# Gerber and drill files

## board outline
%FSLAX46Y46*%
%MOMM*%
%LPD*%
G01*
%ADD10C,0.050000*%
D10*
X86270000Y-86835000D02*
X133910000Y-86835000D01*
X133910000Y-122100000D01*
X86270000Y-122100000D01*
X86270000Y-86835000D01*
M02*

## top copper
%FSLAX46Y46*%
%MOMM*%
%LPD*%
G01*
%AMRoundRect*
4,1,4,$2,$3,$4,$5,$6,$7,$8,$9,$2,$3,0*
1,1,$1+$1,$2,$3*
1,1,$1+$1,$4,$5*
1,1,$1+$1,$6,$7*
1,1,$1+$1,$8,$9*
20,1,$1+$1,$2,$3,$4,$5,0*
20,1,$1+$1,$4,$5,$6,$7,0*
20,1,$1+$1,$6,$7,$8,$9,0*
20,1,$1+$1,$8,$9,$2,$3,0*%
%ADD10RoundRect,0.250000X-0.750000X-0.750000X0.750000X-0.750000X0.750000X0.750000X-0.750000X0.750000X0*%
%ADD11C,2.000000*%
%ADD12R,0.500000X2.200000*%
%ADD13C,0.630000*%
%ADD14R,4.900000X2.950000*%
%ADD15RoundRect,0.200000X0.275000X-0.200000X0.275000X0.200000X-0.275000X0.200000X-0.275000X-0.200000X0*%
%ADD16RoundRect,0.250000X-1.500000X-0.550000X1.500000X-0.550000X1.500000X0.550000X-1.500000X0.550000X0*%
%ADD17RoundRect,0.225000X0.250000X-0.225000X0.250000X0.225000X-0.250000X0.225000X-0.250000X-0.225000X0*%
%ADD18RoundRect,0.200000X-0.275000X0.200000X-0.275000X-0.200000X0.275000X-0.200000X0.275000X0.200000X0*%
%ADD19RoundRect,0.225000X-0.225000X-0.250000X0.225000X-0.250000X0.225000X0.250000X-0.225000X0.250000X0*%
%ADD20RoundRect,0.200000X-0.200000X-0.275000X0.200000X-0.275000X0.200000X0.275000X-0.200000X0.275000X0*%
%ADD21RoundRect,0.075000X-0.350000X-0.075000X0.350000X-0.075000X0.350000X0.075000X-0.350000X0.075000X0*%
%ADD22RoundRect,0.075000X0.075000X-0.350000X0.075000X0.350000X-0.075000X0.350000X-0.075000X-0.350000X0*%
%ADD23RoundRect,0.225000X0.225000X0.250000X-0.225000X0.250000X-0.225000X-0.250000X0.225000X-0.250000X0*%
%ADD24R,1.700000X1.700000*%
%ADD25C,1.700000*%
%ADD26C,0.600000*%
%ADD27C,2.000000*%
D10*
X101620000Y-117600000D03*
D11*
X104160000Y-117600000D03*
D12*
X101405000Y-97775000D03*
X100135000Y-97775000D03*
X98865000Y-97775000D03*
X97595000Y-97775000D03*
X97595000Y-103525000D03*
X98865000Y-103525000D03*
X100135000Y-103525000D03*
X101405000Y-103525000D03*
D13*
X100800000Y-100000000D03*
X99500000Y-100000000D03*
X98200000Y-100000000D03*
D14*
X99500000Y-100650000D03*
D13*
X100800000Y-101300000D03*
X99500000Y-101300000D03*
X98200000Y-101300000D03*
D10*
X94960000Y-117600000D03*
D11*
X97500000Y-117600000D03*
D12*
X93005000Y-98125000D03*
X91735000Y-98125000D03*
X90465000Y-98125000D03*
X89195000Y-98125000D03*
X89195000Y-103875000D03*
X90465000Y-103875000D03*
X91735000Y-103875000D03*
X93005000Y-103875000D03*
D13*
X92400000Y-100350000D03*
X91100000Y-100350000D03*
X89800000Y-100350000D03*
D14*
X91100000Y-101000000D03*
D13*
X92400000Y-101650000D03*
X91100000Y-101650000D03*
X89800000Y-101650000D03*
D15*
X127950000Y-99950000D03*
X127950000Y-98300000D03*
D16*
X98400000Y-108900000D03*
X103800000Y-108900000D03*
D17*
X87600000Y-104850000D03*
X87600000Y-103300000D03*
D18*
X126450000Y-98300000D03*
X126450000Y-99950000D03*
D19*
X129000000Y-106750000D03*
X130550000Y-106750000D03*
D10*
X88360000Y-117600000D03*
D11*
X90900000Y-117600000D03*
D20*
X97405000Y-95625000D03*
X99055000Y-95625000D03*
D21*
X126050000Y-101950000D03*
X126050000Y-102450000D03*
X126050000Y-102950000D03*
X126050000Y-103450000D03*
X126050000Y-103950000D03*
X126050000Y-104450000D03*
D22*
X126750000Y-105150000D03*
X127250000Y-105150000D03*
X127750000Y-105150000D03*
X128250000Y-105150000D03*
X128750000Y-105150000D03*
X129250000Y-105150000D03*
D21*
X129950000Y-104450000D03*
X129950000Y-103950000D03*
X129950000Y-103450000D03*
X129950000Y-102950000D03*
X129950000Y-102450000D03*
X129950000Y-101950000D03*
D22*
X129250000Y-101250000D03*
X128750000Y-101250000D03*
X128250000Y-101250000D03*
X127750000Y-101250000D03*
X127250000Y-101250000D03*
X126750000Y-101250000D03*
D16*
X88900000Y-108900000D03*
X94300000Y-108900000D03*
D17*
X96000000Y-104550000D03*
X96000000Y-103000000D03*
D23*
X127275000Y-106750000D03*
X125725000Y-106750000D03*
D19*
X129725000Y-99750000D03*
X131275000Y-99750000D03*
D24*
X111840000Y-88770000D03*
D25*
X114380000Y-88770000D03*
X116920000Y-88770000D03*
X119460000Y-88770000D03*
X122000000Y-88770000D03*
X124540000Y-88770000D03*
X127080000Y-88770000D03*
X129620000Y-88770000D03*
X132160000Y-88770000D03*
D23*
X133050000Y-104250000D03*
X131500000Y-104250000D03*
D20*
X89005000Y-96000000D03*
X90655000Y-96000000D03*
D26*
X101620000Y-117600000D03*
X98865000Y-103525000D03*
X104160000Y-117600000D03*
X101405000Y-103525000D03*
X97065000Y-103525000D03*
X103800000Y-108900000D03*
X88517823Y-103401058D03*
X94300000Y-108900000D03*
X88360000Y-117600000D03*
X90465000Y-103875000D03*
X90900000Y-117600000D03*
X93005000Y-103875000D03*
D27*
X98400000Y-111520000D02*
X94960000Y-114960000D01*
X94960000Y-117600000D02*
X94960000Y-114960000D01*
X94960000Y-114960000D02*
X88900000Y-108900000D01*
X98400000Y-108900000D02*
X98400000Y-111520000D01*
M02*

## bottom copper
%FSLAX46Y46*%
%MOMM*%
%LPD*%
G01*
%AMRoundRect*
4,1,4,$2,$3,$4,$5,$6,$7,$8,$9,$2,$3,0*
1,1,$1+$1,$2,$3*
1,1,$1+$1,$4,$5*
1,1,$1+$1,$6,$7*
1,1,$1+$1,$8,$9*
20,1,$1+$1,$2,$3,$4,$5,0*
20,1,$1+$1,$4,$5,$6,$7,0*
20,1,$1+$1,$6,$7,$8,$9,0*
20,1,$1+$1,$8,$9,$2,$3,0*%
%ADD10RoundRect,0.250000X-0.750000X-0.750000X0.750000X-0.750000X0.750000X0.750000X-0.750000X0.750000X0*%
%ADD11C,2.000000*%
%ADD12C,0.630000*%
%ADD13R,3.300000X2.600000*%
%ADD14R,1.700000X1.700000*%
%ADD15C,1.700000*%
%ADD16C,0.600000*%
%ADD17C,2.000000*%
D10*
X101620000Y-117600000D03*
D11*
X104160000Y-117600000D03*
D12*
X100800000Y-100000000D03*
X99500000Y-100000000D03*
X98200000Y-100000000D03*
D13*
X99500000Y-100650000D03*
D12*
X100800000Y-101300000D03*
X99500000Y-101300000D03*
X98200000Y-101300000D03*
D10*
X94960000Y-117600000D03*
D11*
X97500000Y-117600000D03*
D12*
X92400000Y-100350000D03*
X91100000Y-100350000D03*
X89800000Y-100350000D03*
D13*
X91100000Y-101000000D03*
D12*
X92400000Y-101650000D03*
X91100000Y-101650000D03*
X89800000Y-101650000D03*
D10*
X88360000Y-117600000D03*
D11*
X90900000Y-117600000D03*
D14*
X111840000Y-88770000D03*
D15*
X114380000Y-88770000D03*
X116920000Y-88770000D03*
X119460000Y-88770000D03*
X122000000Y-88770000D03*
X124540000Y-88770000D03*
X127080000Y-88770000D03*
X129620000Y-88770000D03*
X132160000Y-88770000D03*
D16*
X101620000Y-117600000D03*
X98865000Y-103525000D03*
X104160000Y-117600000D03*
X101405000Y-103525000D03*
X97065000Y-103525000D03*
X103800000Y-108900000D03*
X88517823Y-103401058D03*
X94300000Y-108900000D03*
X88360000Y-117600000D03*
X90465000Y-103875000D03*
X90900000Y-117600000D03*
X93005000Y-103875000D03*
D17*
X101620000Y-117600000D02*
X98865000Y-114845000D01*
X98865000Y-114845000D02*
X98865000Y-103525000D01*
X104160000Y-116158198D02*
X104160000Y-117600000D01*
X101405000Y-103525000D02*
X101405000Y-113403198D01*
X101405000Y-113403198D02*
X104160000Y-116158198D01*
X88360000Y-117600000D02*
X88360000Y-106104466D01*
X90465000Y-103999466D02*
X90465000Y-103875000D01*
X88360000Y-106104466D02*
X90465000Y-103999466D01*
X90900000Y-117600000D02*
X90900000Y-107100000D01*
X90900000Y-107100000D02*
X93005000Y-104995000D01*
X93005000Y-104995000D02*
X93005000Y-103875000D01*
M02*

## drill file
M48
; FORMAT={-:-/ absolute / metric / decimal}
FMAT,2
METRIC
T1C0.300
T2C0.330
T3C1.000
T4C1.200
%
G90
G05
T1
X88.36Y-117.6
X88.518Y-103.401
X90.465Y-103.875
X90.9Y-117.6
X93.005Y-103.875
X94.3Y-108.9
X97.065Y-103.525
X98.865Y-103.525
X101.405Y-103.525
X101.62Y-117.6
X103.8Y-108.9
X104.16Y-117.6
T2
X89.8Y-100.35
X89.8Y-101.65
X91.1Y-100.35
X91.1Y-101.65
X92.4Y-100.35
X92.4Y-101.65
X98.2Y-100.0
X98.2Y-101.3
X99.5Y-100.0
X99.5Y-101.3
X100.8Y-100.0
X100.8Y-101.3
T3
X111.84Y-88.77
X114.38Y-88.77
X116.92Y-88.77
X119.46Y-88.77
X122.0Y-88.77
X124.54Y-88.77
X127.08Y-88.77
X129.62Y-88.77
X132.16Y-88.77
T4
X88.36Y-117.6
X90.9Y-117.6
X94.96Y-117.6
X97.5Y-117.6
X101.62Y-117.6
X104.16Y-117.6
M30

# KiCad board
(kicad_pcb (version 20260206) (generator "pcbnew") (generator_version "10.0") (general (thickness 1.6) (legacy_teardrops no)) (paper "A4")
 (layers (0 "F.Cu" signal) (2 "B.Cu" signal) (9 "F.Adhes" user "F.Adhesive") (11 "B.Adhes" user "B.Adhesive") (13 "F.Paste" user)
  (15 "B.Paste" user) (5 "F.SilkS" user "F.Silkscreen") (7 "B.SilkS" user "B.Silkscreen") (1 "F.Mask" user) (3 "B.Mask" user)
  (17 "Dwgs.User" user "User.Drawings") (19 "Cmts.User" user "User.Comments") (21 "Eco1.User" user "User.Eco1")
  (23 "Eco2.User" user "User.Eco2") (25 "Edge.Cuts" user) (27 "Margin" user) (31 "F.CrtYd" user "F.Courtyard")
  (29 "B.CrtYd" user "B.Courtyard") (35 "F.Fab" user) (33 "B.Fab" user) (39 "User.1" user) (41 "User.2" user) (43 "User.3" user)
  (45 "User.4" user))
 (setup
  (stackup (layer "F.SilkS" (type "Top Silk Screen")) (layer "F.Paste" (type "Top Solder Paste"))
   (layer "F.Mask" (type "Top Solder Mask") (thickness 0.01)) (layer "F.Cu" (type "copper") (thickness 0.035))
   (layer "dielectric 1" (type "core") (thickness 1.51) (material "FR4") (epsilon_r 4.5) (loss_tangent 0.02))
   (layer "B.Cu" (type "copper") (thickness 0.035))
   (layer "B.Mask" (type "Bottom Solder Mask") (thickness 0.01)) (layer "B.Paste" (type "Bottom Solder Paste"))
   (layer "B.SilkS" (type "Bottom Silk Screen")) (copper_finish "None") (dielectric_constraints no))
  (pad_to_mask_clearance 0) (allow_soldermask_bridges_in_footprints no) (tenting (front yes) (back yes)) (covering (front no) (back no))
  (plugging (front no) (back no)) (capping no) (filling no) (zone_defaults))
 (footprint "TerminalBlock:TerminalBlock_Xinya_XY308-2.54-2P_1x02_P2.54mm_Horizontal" (layer "F.Cu") (at 101.62 117.6)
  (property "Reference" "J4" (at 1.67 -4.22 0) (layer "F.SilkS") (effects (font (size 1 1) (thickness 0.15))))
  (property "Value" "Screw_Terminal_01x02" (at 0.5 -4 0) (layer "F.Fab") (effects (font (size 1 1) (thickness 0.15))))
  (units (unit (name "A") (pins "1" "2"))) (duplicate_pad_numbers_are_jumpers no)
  (pad "1" thru_hole roundrect (at 0 0) (size 2 2) (drill 1.2) (layers "*.Cu" "*.Mask") (remove_unused_layers no) (roundrect_rratio 0.125)
   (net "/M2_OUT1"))
  (pad "2" thru_hole circle (at 2.54 0) (size 2 2) (drill 1.2) (layers "*.Cu" "*.Mask") (remove_unused_layers no) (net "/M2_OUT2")))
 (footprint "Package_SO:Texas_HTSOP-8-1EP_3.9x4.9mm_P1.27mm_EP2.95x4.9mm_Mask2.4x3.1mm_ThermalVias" (layer "F.Cu") (at 99.5 100.65 -90)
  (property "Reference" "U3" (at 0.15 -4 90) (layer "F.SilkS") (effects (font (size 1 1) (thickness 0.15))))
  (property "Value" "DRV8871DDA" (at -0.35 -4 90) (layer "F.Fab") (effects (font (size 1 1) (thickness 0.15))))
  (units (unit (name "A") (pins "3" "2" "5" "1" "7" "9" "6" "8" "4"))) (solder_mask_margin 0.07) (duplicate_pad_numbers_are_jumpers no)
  (pad "" smd rect (at 0 0 270) (size 2.4 3.1) (layers "F.Mask"))
  (pad "" smd rect (at 0 0 270) (size 2.4 3.1) (layers "F.Paste"))
  (pad "1" smd rect (at -2.875 -1.905 270) (size 2.2 0.5) (layers "F.Cu" "F.Mask" "F.Paste") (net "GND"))
  (pad "2" smd rect (at -2.875 -0.635 270) (size 2.2 0.5) (layers "F.Cu" "F.Mask" "F.Paste") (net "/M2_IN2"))
  (pad "3" smd rect (at -2.875 0.635 270) (size 2.2 0.5) (layers "F.Cu" "F.Mask" "F.Paste") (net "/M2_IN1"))
  (pad "4" smd rect (at -2.875 1.905 270) (size 2.2 0.5) (layers "F.Cu" "F.Mask" "F.Paste") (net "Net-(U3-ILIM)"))
  (pad "5" smd rect (at 2.875 1.905 270) (size 2.2 0.5) (layers "F.Cu" "F.Mask" "F.Paste") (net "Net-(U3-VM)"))
  (pad "6" smd rect (at 2.875 0.635 270) (size 2.2 0.5) (layers "F.Cu" "F.Mask" "F.Paste") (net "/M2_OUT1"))
  (pad "7" smd rect (at 2.875 -0.635 270) (size 2.2 0.5) (layers "F.Cu" "F.Mask" "F.Paste") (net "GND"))
  (pad "8" smd rect (at 2.875 -1.905 270) (size 2.2 0.5) (layers "F.Cu" "F.Mask" "F.Paste") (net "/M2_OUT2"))
  (pad "9" thru_hole circle (at -0.65 -1.3 270) (size 0.63 0.63) (drill 0.33) (layers "*.Cu" "*.Mask") (remove_unused_layers no) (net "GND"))
  (pad "9" thru_hole circle (at -0.65 0 270) (size 0.63 0.63) (drill 0.33) (layers "*.Cu" "*.Mask") (remove_unused_layers no) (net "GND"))
  (pad "9" thru_hole circle (at -0.65 1.3 270) (size 0.63 0.63) (drill 0.33) (layers "*.Cu" "*.Mask") (remove_unused_layers no) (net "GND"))
  (pad "9" smd rect (at 0 0 270) (size 2.6 3.3) (layers "B.Cu") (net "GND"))
  (pad "9" smd rect (at 0 0 270) (size 2.95 4.9) (layers "F.Cu") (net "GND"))
  (pad "9" thru_hole circle (at 0.65 -1.3 270) (size 0.63 0.63) (drill 0.33) (layers "*.Cu" "*.Mask") (remove_unused_layers no) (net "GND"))
  (pad "9" thru_hole circle (at 0.65 0 270) (size 0.63 0.63) (drill 0.33) (layers "*.Cu" "*.Mask") (remove_unused_layers no) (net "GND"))
  (pad "9" thru_hole circle (at 0.65 1.3 270) (size 0.63 0.63) (drill 0.33) (layers "*.Cu" "*.Mask") (remove_unused_layers no) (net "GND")))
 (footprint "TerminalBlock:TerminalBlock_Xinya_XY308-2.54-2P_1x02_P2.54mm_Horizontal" (layer "F.Cu") (at 94.96 117.6)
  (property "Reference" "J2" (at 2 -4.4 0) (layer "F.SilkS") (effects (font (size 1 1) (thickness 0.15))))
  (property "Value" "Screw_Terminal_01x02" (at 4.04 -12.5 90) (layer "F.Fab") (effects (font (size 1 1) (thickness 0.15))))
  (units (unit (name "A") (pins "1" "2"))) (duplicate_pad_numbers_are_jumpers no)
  (pad "1" thru_hole roundrect (at 0 0) (size 2 2) (drill 1.2) (layers "*.Cu" "*.Mask") (remove_unused_layers no) (roundrect_rratio 0.125)
   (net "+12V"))
  (pad "2" thru_hole circle (at 2.54 0) (size 2 2) (drill 1.2) (layers "*.Cu" "*.Mask") (remove_unused_layers no) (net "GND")))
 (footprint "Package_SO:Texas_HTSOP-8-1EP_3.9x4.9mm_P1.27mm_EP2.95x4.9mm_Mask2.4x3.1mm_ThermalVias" (layer "F.Cu") (at 91.1 101 -90)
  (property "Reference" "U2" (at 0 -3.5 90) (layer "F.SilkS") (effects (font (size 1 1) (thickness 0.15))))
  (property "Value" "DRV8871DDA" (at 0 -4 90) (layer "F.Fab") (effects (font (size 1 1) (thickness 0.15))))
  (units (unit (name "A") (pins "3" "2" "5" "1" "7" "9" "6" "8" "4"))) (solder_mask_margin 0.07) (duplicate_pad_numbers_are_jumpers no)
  (pad "" smd rect (at 0 0 270) (size 2.4 3.1) (layers "F.Mask"))
  (pad "" smd rect (at 0 0 270) (size 2.4 3.1) (layers "F.Paste"))
  (pad "1" smd rect (at -2.875 -1.905 270) (size 2.2 0.5) (layers "F.Cu" "F.Mask" "F.Paste") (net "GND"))
  (pad "2" smd rect (at -2.875 -0.635 270) (size 2.2 0.5) (layers "F.Cu" "F.Mask" "F.Paste") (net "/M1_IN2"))
  (pad "3" smd rect (at -2.875 0.635 270) (size 2.2 0.5) (layers "F.Cu" "F.Mask" "F.Paste") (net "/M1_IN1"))
  (pad "4" smd rect (at -2.875 1.905 270) (size 2.2 0.5) (layers "F.Cu" "F.Mask" "F.Paste") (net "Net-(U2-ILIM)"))
  (pad "5" smd rect (at 2.875 1.905 270) (size 2.2 0.5) (layers "F.Cu" "F.Mask" "F.Paste") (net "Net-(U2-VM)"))
  (pad "6" smd rect (at 2.875 0.635 270) (size 2.2 0.5) (layers "F.Cu" "F.Mask" "F.Paste") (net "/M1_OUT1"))
  (pad "7" smd rect (at 2.875 -0.635 270) (size 2.2 0.5) (layers "F.Cu" "F.Mask" "F.Paste") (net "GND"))
  (pad "8" smd rect (at 2.875 -1.905 270) (size 2.2 0.5) (layers "F.Cu" "F.Mask" "F.Paste") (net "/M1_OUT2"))
  (pad "9" thru_hole circle (at -0.65 -1.3 270) (size 0.63 0.63) (drill 0.33) (layers "*.Cu" "*.Mask") (remove_unused_layers no) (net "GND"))
  (pad "9" thru_hole circle (at -0.65 0 270) (size 0.63 0.63) (drill 0.33) (layers "*.Cu" "*.Mask") (remove_unused_layers no) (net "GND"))
  (pad "9" thru_hole circle (at -0.65 1.3 270) (size 0.63 0.63) (drill 0.33) (layers "*.Cu" "*.Mask") (remove_unused_layers no) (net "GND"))
  (pad "9" smd rect (at 0 0 270) (size 2.6 3.3) (layers "B.Cu") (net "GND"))
  (pad "9" smd rect (at 0 0 270) (size 2.95 4.9) (layers "F.Cu") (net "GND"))
  (pad "9" thru_hole circle (at 0.65 -1.3 270) (size 0.63 0.63) (drill 0.33) (layers "*.Cu" "*.Mask") (remove_unused_layers no) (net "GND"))
  (pad "9" thru_hole circle (at 0.65 0 270) (size 0.63 0.63) (drill 0.33) (layers "*.Cu" "*.Mask") (remove_unused_layers no) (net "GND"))
  (pad "9" thru_hole circle (at 0.65 1.3 270) (size 0.63 0.63) (drill 0.33) (layers "*.Cu" "*.Mask") (remove_unused_layers no) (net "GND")))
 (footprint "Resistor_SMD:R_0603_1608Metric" (layer "F.Cu") (at 127.95 99.125 90)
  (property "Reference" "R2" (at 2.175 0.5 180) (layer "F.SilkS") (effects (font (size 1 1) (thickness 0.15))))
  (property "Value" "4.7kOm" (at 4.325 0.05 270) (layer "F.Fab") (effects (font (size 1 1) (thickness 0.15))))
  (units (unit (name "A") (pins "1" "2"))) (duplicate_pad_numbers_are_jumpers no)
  (pad "1" smd roundrect (at -0.825 0 90) (size 0.8 0.95) (layers "F.Cu" "F.Mask" "F.Paste") (roundrect_rratio 0.25) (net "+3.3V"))
  (pad "2" smd roundrect (at 0.825 0 90) (size 0.8 0.95) (layers "F.Cu" "F.Mask" "F.Paste") (roundrect_rratio 0.25) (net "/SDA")))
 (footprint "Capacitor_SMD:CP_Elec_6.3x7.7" (layer "F.Cu") (at 101.1 108.9)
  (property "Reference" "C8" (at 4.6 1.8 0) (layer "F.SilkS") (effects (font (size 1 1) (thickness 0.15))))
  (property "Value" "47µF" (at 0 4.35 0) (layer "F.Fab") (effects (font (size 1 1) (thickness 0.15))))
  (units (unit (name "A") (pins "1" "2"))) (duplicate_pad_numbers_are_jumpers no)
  (pad "1" smd roundrect (at -2.7 0) (size 3.5 1.6) (layers "F.Cu" "F.Mask" "F.Paste") (roundrect_rratio 0.15625) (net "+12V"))
  (pad "2" smd roundrect (at 2.7 0) (size 3.5 1.6) (layers "F.Cu" "F.Mask" "F.Paste") (roundrect_rratio 0.15625) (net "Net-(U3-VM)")))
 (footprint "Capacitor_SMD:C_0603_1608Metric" (layer "F.Cu") (at 87.6 104.075 90)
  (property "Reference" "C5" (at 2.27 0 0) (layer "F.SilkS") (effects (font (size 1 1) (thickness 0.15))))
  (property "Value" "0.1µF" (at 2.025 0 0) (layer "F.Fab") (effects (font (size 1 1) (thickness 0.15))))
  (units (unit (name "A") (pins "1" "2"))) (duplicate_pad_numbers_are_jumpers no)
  (pad "1" smd roundrect (at -0.775 0 90) (size 0.9 0.95) (layers "F.Cu" "F.Mask" "F.Paste") (roundrect_rratio 0.25) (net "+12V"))
  (pad "2" smd roundrect (at 0.775 0 90) (size 0.9 0.95) (layers "F.Cu" "F.Mask" "F.Paste") (roundrect_rratio 0.25) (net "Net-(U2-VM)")))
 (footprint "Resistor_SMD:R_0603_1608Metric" (layer "F.Cu") (at 126.45 99.125 -90)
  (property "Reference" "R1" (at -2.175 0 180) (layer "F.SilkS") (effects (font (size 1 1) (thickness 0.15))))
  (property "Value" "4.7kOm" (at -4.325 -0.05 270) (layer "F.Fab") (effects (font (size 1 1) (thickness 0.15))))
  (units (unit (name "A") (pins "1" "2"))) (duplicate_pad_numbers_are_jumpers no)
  (pad "1" smd roundrect (at -0.825 0 270) (size 0.8 0.95) (layers "F.Cu" "F.Mask" "F.Paste") (roundrect_rratio 0.25) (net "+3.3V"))
  (pad "2" smd roundrect (at 0.825 0 270) (size 0.8 0.95) (layers "F.Cu" "F.Mask" "F.Paste") (roundrect_rratio 0.25) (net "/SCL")))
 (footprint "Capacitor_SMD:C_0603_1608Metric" (layer "F.Cu") (at 129.775 106.75)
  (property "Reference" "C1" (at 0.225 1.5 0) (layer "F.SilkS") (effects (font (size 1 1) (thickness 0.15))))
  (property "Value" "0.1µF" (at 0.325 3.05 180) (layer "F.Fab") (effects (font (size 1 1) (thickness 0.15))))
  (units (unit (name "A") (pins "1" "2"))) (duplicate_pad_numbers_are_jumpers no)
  (pad "1" smd roundrect (at -0.775 0) (size 0.9 0.95) (layers "F.Cu" "F.Mask" "F.Paste") (roundrect_rratio 0.25) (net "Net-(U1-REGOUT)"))
  (pad "2" smd roundrect (at 0.775 0) (size 0.9 0.95) (layers "F.Cu" "F.Mask" "F.Paste") (roundrect_rratio 0.25) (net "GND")))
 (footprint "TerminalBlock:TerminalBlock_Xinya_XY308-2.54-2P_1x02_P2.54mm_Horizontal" (layer "F.Cu") (at 88.36 117.6)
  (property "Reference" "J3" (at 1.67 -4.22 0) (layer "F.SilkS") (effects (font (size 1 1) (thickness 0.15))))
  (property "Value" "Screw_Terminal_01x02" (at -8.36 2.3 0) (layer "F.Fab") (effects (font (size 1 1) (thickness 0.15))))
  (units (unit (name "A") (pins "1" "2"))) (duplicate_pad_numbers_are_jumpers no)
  (pad "1" thru_hole roundrect (at 0 0) (size 2 2) (drill 1.2) (layers "*.Cu" "*.Mask") (remove_unused_layers no) (roundrect_rratio 0.125)
   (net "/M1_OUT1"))
  (pad "2" thru_hole circle (at 2.54 0) (size 2 2) (drill 1.2) (layers "*.Cu" "*.Mask") (remove_unused_layers no) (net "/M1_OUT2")))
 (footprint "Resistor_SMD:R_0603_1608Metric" (layer "F.Cu") (at 98.23 95.625)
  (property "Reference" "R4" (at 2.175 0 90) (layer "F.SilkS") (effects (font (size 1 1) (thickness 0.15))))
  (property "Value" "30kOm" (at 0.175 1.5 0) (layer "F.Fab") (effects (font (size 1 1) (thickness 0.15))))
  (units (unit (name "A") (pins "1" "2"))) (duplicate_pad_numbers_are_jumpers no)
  (pad "1" smd roundrect (at -0.825 0) (size 0.8 0.95) (layers "F.Cu" "F.Mask" "F.Paste") (roundrect_rratio 0.25) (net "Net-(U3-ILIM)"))
  (pad "2" smd roundrect (at 0.825 0) (size 0.8 0.95) (layers "F.Cu" "F.Mask" "F.Paste") (roundrect_rratio 0.25) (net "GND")))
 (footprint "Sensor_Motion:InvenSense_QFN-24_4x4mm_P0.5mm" (layer "F.Cu") (at 128 103.2)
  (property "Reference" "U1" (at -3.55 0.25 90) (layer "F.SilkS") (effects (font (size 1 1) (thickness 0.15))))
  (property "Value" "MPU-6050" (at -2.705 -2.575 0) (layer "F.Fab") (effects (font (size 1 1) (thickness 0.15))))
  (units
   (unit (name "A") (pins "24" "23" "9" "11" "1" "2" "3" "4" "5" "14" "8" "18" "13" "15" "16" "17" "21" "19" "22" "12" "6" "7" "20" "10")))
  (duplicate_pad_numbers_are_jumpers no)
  (pad "1" smd roundrect (at -1.95 -1.25) (size 0.85 0.3) (layers "F.Cu" "F.Mask" "F.Paste") (roundrect_rratio 0.25) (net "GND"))
  (pad "2" smd roundrect (at -1.95 -0.75) (size 0.85 0.3) (layers "F.Cu" "F.Mask" "F.Paste") (roundrect_rratio 0.25)
   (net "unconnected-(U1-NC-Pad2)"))
  (pad "3" smd roundrect (at -1.95 -0.25) (size 0.85 0.3) (layers "F.Cu" "F.Mask" "F.Paste") (roundrect_rratio 0.25)
   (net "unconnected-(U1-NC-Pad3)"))
  (pad "4" smd roundrect (at -1.95 0.25) (size 0.85 0.3) (layers "F.Cu" "F.Mask" "F.Paste") (roundrect_rratio 0.25)
   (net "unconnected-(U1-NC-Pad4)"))
  (pad "5" smd roundrect (at -1.95 0.75) (size 0.85 0.3) (layers "F.Cu" "F.Mask" "F.Paste") (roundrect_rratio 0.25)
   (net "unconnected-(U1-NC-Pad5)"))
  (pad "6" smd roundrect (at -1.95 1.25) (size 0.85 0.3) (layers "F.Cu" "F.Mask" "F.Paste") (roundrect_rratio 0.25)
   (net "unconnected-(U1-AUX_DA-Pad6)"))
  (pad "7" smd roundrect (at -1.25 1.95 90) (size 0.85 0.3) (layers "F.Cu" "F.Mask" "F.Paste") (roundrect_rratio 0.25)
   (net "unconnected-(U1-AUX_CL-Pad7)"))
  (pad "8" smd roundrect (at -0.75 1.95 90) (size 0.85 0.3) (layers "F.Cu" "F.Mask" "F.Paste") (roundrect_rratio 0.25)
   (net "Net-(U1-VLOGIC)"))
  (pad "9" smd roundrect (at -0.25 1.95 90) (size 0.85 0.3) (layers "F.Cu" "F.Mask" "F.Paste") (roundrect_rratio 0.25) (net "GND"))
  (pad "10" smd roundrect (at 0.25 1.95 90) (size 0.85 0.3) (layers "F.Cu" "F.Mask" "F.Paste") (roundrect_rratio 0.25)
   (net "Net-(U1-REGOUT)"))
  (pad "11" smd roundrect (at 0.75 1.95 90) (size 0.85 0.3) (layers "F.Cu" "F.Mask" "F.Paste") (roundrect_rratio 0.25) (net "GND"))
  (pad "12" smd roundrect (at 1.25 1.95 90) (size 0.85 0.3) (layers "F.Cu" "F.Mask" "F.Paste") (roundrect_rratio 0.25) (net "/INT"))
  (pad "13" smd roundrect (at 1.95 1.25) (size 0.85 0.3) (layers "F.Cu" "F.Mask" "F.Paste") (roundrect_rratio 0.25) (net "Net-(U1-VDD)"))
  (pad "14" smd roundrect (at 1.95 0.75) (size 0.85 0.3) (layers "F.Cu" "F.Mask" "F.Paste") (roundrect_rratio 0.25)
   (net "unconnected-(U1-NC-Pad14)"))
  (pad "15" smd roundrect (at 1.95 0.25) (size 0.85 0.3) (layers "F.Cu" "F.Mask" "F.Paste") (roundrect_rratio 0.25)
   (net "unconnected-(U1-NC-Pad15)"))
  (pad "16" smd roundrect (at 1.95 -0.25) (size 0.85 0.3) (layers "F.Cu" "F.Mask" "F.Paste") (roundrect_rratio 0.25)
   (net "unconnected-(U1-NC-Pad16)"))
  (pad "17" smd roundrect (at 1.95 -0.75) (size 0.85 0.3) (layers "F.Cu" "F.Mask" "F.Paste") (roundrect_rratio 0.25)
   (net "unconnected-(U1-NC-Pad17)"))
  (pad "18" smd roundrect (at 1.95 -1.25) (size 0.85 0.3) (layers "F.Cu" "F.Mask" "F.Paste") (roundrect_rratio 0.25) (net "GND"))
  (pad "19" smd roundrect (at 1.25 -1.95 90) (size 0.85 0.3) (layers "F.Cu" "F.Mask" "F.Paste") (roundrect_rratio 0.25)
   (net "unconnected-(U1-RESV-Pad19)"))
  (pad "20" smd roundrect (at 0.75 -1.95 90) (size 0.85 0.3) (layers "F.Cu" "F.Mask" "F.Paste") (roundrect_rratio 0.25)
   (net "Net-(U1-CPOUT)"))
  (pad "21" smd roundrect (at 0.25 -1.95 90) (size 0.85 0.3) (layers "F.Cu" "F.Mask" "F.Paste") (roundrect_rratio 0.25)
   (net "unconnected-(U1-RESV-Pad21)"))
  (pad "22" smd roundrect (at -0.25 -1.95 90) (size 0.85 0.3) (layers "F.Cu" "F.Mask" "F.Paste") (roundrect_rratio 0.25)
   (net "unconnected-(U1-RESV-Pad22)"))
  (pad "23" smd roundrect (at -0.75 -1.95 90) (size 0.85 0.3) (layers "F.Cu" "F.Mask" "F.Paste") (roundrect_rratio 0.25) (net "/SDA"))
  (pad "24" smd roundrect (at -1.25 -1.95 90) (size 0.85 0.3) (layers "F.Cu" "F.Mask" "F.Paste") (roundrect_rratio 0.25) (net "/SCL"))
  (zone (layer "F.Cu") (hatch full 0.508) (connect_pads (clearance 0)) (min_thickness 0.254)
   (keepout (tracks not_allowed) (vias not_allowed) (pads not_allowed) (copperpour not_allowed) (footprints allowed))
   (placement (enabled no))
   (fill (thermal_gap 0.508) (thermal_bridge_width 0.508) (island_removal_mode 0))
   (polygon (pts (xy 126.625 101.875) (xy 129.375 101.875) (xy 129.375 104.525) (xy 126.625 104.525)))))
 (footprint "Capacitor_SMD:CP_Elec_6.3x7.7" (layer "F.Cu") (at 91.6 108.9)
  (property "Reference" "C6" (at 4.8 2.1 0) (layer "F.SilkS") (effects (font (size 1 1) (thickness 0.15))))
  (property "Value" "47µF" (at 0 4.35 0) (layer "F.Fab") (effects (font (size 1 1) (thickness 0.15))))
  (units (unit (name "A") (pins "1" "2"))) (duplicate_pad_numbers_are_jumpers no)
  (pad "1" smd roundrect (at -2.7 0) (size 3.5 1.6) (layers "F.Cu" "F.Mask" "F.Paste") (roundrect_rratio 0.15625) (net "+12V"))
  (pad "2" smd roundrect (at 2.7 0) (size 3.5 1.6) (layers "F.Cu" "F.Mask" "F.Paste") (roundrect_rratio 0.15625) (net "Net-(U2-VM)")))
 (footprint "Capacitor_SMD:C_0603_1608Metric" (layer "F.Cu") (at 96 103.775 90)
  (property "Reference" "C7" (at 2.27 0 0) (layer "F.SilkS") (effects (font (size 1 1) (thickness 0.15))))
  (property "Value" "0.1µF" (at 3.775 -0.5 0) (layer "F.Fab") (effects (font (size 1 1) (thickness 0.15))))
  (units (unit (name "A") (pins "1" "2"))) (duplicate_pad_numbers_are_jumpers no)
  (pad "1" smd roundrect (at -0.775 0 90) (size 0.9 0.95) (layers "F.Cu" "F.Mask" "F.Paste") (roundrect_rratio 0.25) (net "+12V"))
  (pad "2" smd roundrect (at 0.775 0 90) (size 0.9 0.95) (layers "F.Cu" "F.Mask" "F.Paste") (roundrect_rratio 0.25) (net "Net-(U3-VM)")))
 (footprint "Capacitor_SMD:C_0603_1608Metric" (layer "F.Cu") (at 126.5 106.75 180)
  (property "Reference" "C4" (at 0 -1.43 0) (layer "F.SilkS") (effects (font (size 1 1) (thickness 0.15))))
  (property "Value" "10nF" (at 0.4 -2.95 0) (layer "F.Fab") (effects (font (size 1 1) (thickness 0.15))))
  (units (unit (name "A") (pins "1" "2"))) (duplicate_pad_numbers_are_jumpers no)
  (pad "1" smd roundrect (at -0.775 0 180) (size 0.9 0.95) (layers "F.Cu" "F.Mask" "F.Paste") (roundrect_rratio 0.25) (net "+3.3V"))
  (pad "2" smd roundrect (at 0.775 0 180) (size 0.9 0.95) (layers "F.Cu" "F.Mask" "F.Paste") (roundrect_rratio 0.25) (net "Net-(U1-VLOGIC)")))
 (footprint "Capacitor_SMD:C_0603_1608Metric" (layer "F.Cu") (at 130.5 99.75)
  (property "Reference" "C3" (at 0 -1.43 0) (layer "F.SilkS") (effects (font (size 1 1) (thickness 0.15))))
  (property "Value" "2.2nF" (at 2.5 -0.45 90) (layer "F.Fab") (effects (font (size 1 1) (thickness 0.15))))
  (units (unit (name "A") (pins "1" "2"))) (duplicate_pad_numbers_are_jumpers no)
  (pad "1" smd roundrect (at -0.775 0) (size 0.9 0.95) (layers "F.Cu" "F.Mask" "F.Paste") (roundrect_rratio 0.25) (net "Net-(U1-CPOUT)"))
  (pad "2" smd roundrect (at 0.775 0) (size 0.9 0.95) (layers "F.Cu" "F.Mask" "F.Paste") (roundrect_rratio 0.25) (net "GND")))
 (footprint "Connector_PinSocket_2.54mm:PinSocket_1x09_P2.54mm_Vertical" (layer "F.Cu") (at 111.84 88.77 90)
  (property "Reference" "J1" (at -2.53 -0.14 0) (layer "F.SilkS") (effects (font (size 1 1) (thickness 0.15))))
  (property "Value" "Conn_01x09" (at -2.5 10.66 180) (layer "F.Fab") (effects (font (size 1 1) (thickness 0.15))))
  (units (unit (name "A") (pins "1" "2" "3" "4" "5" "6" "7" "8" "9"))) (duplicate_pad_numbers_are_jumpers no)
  (pad "1" thru_hole rect (at 0 0 90) (size 1.7 1.7) (drill 1) (layers "*.Cu" "*.Mask") (remove_unused_layers no) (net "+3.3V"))
  (pad "2" thru_hole circle (at 0 2.54 90) (size 1.7 1.7) (drill 1) (layers "*.Cu" "*.Mask") (remove_unused_layers no) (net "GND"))
  (pad "3" thru_hole circle (at 0 5.08 90) (size 1.7 1.7) (drill 1) (layers "*.Cu" "*.Mask") (remove_unused_layers no) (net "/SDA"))
  (pad "4" thru_hole circle (at 0 7.62 90) (size 1.7 1.7) (drill 1) (layers "*.Cu" "*.Mask") (remove_unused_layers no) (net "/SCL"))
  (pad "5" thru_hole circle (at 0 10.16 90) (size 1.7 1.7) (drill 1) (layers "*.Cu" "*.Mask") (remove_unused_layers no) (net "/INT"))
  (pad "6" thru_hole circle (at 0 12.7 90) (size 1.7 1.7) (drill 1) (layers "*.Cu" "*.Mask") (remove_unused_layers no) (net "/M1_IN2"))
  (pad "7" thru_hole circle (at 0 15.24 90) (size 1.7 1.7) (drill 1) (layers "*.Cu" "*.Mask") (remove_unused_layers no) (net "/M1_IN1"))
  (pad "8" thru_hole circle (at 0 17.78 90) (size 1.7 1.7) (drill 1) (layers "*.Cu" "*.Mask") (remove_unused_layers no) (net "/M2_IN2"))
  (pad "9" thru_hole circle (at 0 20.32 90) (size 1.7 1.7) (drill 1) (layers "*.Cu" "*.Mask") (remove_unused_layers no) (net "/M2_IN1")))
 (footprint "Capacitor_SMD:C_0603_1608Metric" (layer "F.Cu") (at 132.275 104.25 180)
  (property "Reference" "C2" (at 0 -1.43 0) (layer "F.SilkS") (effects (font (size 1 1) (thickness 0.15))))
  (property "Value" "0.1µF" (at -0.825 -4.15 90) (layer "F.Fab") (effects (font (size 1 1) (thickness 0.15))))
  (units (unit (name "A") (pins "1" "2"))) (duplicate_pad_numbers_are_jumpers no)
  (pad "1" smd roundrect (at -0.775 0 180) (size 0.9 0.95) (layers "F.Cu" "F.Mask" "F.Paste") (roundrect_rratio 0.25) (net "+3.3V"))
  (pad "2" smd roundrect (at 0.775 0 180) (size 0.9 0.95) (layers "F.Cu" "F.Mask" "F.Paste") (roundrect_rratio 0.25) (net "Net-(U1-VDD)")))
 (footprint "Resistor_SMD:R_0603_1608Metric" (layer "F.Cu") (at 89.83 96)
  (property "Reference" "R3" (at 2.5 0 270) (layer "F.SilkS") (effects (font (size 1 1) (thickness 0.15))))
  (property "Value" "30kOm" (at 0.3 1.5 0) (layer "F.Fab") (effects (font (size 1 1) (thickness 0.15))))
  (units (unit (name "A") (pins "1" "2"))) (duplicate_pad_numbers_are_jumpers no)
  (pad "1" smd roundrect (at -0.825 0) (size 0.8 0.95) (layers "F.Cu" "F.Mask" "F.Paste") (roundrect_rratio 0.25) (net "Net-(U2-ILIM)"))
  (pad "2" smd roundrect (at 0.825 0) (size 0.8 0.95) (layers "F.Cu" "F.Mask" "F.Paste") (roundrect_rratio 0.25) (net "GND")))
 (gr_rect (start 86.27 86.835) (end 133.91 122.1) (stroke (width 0.05) (type default)) (fill no) (layer "Edge.Cuts"))
 (via (at 101.62 117.6) (size 0.6) (drill 0.3) (layers "F.Cu" "B.Cu") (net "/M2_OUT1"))
 (via (at 98.865 103.525) (size 0.6) (drill 0.3) (layers "F.Cu" "B.Cu") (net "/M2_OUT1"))
 (segment (start 101.62 117.6) (end 98.865 114.845) (width 2) (layer "B.Cu") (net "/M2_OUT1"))
 (segment (start 98.865 114.845) (end 98.865 103.525) (width 2) (layer "B.Cu") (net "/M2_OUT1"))
 (via (at 104.16 117.6) (size 0.6) (drill 0.3) (layers "F.Cu" "B.Cu") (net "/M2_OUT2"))
 (via (at 101.405 103.525) (size 0.6) (drill 0.3) (layers "F.Cu" "B.Cu") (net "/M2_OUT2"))
 (segment (start 104.16 116.158198) (end 104.16 117.6) (width 2) (layer "B.Cu") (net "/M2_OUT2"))
 (segment (start 101.405 103.525) (end 101.405 113.403198) (width 2) (layer "B.Cu") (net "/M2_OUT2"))
 (segment (start 101.405 113.403198) (end 104.16 116.158198) (width 2) (layer "B.Cu") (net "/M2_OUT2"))
 (via (at 97.065 103.525) (size 0.6) (drill 0.3) (layers "F.Cu" "B.Cu") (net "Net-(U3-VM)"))
 (via (at 103.8 108.9) (size 0.6) (drill 0.3) (layers "F.Cu" "B.Cu") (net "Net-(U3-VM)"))
 (segment (start 98.4 111.52) (end 94.96 114.96) (width 2) (layer "F.Cu") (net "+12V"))
 (segment (start 94.96 117.6) (end 94.96 114.96) (width 2) (layer "F.Cu") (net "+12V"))
 (segment (start 94.96 114.96) (end 88.9 108.9) (width 2) (layer "F.Cu") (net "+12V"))
 (segment (start 98.4 108.9) (end 98.4 111.52) (width 2) (layer "F.Cu") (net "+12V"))
 (via (at 88.517823 103.401058) (size 0.6) (drill 0.3) (layers "F.Cu" "B.Cu") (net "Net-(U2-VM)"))
 (via (at 94.3 108.9) (size 0.6) (drill 0.3) (layers "F.Cu" "B.Cu") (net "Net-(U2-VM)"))
 (via (at 88.36 117.6) (size 0.6) (drill 0.3) (layers "F.Cu" "B.Cu") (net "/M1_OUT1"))
 (via (at 90.465 103.875) (size 0.6) (drill 0.3) (layers "F.Cu" "B.Cu") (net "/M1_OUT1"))
 (segment (start 88.36 117.6) (end 88.36 106.104466) (width 2) (layer "B.Cu") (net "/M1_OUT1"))
 (segment (start 90.465 103.999466) (end 90.465 103.875) (width 2) (layer "B.Cu") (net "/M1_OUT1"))
 (segment (start 88.36 106.104466) (end 90.465 103.999466) (width 2) (layer "B.Cu") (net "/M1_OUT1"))
 (via (at 90.9 117.6) (size 0.6) (drill 0.3) (layers "F.Cu" "B.Cu") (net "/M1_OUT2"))
 (via (at 93.005 103.875) (size 0.6) (drill 0.3) (layers "F.Cu" "B.Cu") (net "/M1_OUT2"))
 (segment (start 90.9 117.6) (end 90.9 107.1) (width 2) (layer "B.Cu") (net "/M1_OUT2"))
 (segment (start 90.9 107.1) (end 93.005 104.995) (width 2) (layer "B.Cu") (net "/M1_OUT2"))
 (segment (start 93.005 104.995) (end 93.005 103.875) (width 2) (layer "B.Cu") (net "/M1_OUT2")))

